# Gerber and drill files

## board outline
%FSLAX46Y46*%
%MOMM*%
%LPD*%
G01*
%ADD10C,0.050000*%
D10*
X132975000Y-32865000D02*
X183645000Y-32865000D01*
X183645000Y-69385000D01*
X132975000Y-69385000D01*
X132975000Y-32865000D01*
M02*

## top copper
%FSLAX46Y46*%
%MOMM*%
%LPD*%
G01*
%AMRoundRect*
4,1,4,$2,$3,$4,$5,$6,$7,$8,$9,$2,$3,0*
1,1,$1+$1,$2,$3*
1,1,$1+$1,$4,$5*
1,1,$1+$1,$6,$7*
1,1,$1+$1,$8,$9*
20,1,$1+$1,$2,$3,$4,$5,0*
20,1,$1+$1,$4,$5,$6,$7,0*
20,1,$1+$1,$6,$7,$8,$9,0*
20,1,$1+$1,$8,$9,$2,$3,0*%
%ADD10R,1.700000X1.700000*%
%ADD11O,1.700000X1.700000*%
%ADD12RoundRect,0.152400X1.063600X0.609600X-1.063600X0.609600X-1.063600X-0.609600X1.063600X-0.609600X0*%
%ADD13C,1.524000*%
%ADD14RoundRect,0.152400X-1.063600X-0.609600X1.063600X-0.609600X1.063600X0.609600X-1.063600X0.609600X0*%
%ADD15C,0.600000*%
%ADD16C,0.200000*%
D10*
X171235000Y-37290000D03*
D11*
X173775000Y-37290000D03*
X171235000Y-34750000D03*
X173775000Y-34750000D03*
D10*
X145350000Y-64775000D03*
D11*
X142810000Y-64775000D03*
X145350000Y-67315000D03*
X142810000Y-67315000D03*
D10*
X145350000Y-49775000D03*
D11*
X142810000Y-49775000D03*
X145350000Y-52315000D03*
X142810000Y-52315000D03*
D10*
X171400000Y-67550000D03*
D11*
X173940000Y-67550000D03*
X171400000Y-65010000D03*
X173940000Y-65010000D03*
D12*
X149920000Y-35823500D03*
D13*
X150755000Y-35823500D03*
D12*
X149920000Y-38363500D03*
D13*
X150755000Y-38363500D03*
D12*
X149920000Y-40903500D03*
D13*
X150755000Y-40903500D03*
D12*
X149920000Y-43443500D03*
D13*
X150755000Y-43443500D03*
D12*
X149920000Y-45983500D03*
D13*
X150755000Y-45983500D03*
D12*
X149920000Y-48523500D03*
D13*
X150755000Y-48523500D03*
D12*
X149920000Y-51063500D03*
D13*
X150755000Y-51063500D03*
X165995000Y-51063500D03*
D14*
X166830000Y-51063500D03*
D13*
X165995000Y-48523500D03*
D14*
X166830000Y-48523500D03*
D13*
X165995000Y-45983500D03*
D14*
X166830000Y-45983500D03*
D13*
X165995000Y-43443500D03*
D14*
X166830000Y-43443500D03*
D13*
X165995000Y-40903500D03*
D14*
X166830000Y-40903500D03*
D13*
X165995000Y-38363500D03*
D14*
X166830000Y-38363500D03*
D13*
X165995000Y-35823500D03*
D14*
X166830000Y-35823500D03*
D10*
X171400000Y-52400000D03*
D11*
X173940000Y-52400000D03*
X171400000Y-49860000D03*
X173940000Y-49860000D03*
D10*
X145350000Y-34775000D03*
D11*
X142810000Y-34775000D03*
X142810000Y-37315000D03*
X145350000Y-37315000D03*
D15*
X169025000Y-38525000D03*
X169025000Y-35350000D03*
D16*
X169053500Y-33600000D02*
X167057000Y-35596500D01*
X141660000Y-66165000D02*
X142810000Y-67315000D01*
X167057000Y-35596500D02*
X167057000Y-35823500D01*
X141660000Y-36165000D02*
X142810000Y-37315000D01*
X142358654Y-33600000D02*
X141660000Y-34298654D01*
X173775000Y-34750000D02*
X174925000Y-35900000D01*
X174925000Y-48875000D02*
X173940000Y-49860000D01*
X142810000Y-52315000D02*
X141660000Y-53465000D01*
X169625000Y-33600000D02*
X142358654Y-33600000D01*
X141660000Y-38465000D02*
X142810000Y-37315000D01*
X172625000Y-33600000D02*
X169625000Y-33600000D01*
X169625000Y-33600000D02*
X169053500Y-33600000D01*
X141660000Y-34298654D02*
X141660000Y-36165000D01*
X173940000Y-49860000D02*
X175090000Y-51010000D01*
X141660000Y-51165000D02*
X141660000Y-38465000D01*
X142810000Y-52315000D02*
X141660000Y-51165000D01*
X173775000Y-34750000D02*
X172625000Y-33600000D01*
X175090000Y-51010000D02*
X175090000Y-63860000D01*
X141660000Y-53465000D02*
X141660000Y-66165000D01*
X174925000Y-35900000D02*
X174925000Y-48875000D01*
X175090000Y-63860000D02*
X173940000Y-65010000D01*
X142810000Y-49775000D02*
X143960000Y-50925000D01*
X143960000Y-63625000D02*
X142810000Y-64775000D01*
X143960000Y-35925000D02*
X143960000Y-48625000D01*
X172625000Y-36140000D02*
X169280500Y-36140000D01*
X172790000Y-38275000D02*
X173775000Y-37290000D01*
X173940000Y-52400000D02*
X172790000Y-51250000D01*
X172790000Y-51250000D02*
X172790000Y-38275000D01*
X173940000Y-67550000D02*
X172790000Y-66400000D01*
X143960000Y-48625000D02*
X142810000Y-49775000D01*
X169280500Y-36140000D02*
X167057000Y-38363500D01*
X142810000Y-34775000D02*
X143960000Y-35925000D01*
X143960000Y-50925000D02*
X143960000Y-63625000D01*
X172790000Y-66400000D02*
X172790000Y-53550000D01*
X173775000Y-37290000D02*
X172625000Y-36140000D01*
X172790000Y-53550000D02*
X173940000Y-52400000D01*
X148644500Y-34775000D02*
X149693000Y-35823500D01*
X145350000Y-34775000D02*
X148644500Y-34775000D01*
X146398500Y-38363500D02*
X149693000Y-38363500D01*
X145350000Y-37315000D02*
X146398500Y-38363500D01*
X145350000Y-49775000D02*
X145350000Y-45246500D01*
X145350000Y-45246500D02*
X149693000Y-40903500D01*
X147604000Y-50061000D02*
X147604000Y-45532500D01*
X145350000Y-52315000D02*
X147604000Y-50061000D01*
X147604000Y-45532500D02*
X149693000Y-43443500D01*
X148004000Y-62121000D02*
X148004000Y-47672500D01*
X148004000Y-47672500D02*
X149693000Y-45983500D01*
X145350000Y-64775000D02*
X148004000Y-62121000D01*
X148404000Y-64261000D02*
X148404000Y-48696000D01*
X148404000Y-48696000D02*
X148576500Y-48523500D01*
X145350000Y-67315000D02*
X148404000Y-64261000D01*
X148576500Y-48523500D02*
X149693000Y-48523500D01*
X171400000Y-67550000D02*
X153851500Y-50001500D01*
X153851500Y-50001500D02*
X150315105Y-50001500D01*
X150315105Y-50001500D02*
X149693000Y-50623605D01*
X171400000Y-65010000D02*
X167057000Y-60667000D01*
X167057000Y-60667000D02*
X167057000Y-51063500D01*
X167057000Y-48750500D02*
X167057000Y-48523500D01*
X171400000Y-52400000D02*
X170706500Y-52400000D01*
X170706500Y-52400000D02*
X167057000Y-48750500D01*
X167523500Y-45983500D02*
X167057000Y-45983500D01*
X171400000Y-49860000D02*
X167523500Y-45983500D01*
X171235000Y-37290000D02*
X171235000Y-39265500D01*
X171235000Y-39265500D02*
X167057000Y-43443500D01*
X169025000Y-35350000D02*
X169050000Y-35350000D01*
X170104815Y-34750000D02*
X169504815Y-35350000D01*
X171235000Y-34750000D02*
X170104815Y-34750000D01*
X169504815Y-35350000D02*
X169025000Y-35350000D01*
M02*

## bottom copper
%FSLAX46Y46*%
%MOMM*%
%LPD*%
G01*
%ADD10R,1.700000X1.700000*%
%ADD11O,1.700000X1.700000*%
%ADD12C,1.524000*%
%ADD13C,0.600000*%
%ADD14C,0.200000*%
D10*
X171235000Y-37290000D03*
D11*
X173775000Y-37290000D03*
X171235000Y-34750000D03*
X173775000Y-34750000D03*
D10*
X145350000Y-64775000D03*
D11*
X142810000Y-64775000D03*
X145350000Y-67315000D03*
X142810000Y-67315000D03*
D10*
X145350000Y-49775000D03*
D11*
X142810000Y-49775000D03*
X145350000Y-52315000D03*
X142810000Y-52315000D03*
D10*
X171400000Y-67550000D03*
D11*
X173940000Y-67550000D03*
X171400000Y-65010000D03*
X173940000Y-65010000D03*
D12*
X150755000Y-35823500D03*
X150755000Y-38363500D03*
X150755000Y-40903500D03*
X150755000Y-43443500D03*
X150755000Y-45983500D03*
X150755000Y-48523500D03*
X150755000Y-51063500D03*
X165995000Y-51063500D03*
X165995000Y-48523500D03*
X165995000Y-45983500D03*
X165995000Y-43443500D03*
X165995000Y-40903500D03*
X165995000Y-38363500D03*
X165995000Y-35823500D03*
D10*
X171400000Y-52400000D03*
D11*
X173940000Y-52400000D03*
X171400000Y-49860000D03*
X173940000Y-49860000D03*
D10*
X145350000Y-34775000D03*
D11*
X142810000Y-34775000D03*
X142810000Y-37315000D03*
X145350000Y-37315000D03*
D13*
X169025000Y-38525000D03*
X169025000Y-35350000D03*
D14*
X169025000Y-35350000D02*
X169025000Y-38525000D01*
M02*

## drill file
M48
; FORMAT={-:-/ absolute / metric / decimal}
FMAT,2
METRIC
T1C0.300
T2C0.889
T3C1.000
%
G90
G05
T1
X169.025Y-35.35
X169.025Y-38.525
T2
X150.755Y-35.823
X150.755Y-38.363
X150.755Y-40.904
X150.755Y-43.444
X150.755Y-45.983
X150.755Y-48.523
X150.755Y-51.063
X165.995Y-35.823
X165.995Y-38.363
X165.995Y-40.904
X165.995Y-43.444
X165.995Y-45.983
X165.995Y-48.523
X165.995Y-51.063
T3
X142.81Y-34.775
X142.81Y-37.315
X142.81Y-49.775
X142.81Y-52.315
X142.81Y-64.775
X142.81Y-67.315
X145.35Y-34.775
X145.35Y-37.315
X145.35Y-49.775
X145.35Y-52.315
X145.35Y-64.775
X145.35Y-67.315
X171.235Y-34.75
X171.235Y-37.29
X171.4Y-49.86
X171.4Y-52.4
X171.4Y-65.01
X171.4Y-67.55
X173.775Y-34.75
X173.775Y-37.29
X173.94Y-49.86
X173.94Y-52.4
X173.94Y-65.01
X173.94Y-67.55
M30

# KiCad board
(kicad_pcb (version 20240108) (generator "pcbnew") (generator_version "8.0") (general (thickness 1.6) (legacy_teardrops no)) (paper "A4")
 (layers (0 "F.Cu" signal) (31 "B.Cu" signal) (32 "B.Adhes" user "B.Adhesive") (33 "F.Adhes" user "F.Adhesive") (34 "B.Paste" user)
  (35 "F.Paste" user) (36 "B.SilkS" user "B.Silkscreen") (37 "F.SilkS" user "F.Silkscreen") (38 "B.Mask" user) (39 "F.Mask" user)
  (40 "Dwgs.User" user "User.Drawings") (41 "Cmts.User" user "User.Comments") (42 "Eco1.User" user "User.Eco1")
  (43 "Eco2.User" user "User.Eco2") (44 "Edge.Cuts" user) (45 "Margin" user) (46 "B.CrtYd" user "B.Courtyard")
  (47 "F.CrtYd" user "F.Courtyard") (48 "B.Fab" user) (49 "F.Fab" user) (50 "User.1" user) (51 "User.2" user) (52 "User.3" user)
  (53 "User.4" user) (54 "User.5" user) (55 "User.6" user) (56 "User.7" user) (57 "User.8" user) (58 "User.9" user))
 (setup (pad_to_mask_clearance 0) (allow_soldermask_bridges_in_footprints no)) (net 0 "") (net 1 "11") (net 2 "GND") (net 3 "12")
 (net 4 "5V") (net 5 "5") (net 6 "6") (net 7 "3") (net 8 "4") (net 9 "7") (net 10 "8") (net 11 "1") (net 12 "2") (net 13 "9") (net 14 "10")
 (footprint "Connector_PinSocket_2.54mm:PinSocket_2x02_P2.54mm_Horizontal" (layer "F.Cu") (at 171.235 37.29 180)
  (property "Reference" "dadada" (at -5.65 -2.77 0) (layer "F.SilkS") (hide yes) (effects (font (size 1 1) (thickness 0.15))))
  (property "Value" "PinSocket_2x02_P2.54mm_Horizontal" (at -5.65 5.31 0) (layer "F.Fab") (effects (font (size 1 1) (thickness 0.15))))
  (pad "1" thru_hole rect (at 0 0 180) (size 1.7 1.7) (drill 1) (layers "*.Cu" "*.Mask") (remove_unused_layers no) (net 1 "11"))
  (pad "2" thru_hole oval (at -2.54 0 180) (size 1.7 1.7) (drill 1) (layers "*.Cu" "*.Mask") (remove_unused_layers no) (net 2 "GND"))
  (pad "3" thru_hole oval (at 0 2.54 180) (size 1.7 1.7) (drill 1) (layers "*.Cu" "*.Mask") (remove_unused_layers no) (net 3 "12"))
  (pad "4" thru_hole oval (at -2.54 2.54 180) (size 1.7 1.7) (drill 1) (layers "*.Cu" "*.Mask") (remove_unused_layers no) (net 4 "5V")))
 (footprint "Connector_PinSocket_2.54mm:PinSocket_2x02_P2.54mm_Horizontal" (layer "F.Cu") (at 145.35 64.775)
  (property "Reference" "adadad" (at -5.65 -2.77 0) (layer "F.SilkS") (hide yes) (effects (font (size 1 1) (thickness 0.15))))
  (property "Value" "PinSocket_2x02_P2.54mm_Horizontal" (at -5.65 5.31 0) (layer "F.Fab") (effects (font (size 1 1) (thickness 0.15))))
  (pad "1" thru_hole rect (at 0 0) (size 1.7 1.7) (drill 1) (layers "*.Cu" "*.Mask") (remove_unused_layers no) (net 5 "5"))
  (pad "2" thru_hole oval (at -2.54 0) (size 1.7 1.7) (drill 1) (layers "*.Cu" "*.Mask") (remove_unused_layers no) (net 2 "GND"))
  (pad "3" thru_hole oval (at 0 2.54) (size 1.7 1.7) (drill 1) (layers "*.Cu" "*.Mask") (remove_unused_layers no) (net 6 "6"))
  (pad "4" thru_hole oval (at -2.54 2.54) (size 1.7 1.7) (drill 1) (layers "*.Cu" "*.Mask") (remove_unused_layers no) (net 4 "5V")))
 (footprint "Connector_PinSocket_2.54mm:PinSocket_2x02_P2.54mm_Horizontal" (layer "F.Cu") (at 145.35 49.775)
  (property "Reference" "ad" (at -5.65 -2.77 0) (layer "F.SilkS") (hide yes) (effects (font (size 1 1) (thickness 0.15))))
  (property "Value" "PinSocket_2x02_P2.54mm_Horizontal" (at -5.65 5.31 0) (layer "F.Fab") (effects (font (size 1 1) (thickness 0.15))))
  (pad "1" thru_hole rect (at 0 0) (size 1.7 1.7) (drill 1) (layers "*.Cu" "*.Mask") (remove_unused_layers no) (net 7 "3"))
  (pad "2" thru_hole oval (at -2.54 0) (size 1.7 1.7) (drill 1) (layers "*.Cu" "*.Mask") (remove_unused_layers no) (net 2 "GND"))
  (pad "3" thru_hole oval (at 0 2.54) (size 1.7 1.7) (drill 1) (layers "*.Cu" "*.Mask") (remove_unused_layers no) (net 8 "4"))
  (pad "4" thru_hole oval (at -2.54 2.54) (size 1.7 1.7) (drill 1) (layers "*.Cu" "*.Mask") (remove_unused_layers no) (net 4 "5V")))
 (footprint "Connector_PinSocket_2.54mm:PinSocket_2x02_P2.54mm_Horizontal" (layer "F.Cu") (at 171.4 67.55 180)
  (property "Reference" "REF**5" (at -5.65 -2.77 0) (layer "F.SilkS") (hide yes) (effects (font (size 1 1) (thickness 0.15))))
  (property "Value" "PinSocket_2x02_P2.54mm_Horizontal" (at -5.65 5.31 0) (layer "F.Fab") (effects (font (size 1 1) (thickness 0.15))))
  (pad "1" thru_hole rect (at 0 0 180) (size 1.7 1.7) (drill 1) (layers "*.Cu" "*.Mask") (remove_unused_layers no) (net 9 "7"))
  (pad "2" thru_hole oval (at -2.54 0 180) (size 1.7 1.7) (drill 1) (layers "*.Cu" "*.Mask") (remove_unused_layers no) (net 2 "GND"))
  (pad "3" thru_hole oval (at 0 2.54 180) (size 1.7 1.7) (drill 1) (layers "*.Cu" "*.Mask") (remove_unused_layers no) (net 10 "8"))
  (pad "4" thru_hole oval (at -2.54 2.54 180) (size 1.7 1.7) (drill 1) (layers "*.Cu" "*.Mask" "B.Paste") (remove_unused_layers no)
   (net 4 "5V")))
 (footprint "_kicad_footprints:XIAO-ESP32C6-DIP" (layer "F.Cu") (at 158.42 43.4435)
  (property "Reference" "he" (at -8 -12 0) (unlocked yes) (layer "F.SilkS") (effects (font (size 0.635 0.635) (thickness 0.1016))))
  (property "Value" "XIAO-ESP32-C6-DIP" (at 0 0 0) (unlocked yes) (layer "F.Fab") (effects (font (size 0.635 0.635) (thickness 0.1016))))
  (pad "1" smd roundrect (at -8.5 -7.62 180) (size 2.432 1.524) (layers "F.Cu" "F.Mask") (roundrect_rratio 0.1) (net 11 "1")
   (thermal_bridge_angle 45))
  (pad "1" thru_hole circle (at -7.665 -7.62 180) (size 1.524 1.524) (drill 0.889) (layers "*.Cu" "*.Mask") (remove_unused_layers no))
  (pad "2" smd roundrect (at -8.5 -5.08 180) (size 2.432 1.524) (layers "F.Cu" "F.Mask") (roundrect_rratio 0.1) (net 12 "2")
   (thermal_bridge_angle 45))
  (pad "2" thru_hole circle (at -7.665 -5.08 180) (size 1.524 1.524) (drill 0.889) (layers "*.Cu" "*.Mask") (remove_unused_layers no))
  (pad "3" smd roundrect (at -8.5 -2.54 180) (size 2.432 1.524) (layers "F.Cu" "F.Mask") (roundrect_rratio 0.1) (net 7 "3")
   (thermal_bridge_angle 45))
  (pad "3" thru_hole circle (at -7.665 -2.54 180) (size 1.524 1.524) (drill 0.889) (layers "*.Cu" "*.Mask") (remove_unused_layers no))
  (pad "4" smd roundrect (at -8.5 0 180) (size 2.432 1.524) (layers "F.Cu" "F.Mask") (roundrect_rratio 0.1) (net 8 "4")
   (thermal_bridge_angle 45))
  (pad "4" thru_hole circle (at -7.665 0 180) (size 1.524 1.524) (drill 0.889) (layers "*.Cu" "*.Mask") (remove_unused_layers no))
  (pad "5" smd roundrect (at -8.5 2.54 180) (size 2.432 1.524) (layers "F.Cu" "F.Mask") (roundrect_rratio 0.1) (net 5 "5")
   (thermal_bridge_angle 45))
  (pad "5" thru_hole circle (at -7.665 2.54 180) (size 1.524 1.524) (drill 0.889) (layers "*.Cu" "*.Mask") (remove_unused_layers no))
  (pad "6" smd roundrect (at -8.5 5.08 180) (size 2.432 1.524) (layers "F.Cu" "F.Mask") (roundrect_rratio 0.1) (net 6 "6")
   (thermal_bridge_angle 45))
  (pad "6" thru_hole circle (at -7.665 5.08 180) (size 1.524 1.524) (drill 0.889) (layers "*.Cu" "*.Mask") (remove_unused_layers no))
  (pad "7" smd roundrect (at -8.5 7.62 180) (size 2.432 1.524) (layers "F.Cu" "F.Mask") (roundrect_rratio 0.1) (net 9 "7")
   (thermal_bridge_angle 45))
  (pad "7" thru_hole circle (at -7.665 7.62 180) (size 1.524 1.524) (drill 0.889) (layers "*.Cu" "*.Mask") (remove_unused_layers no))
  (pad "8" thru_hole circle (at 7.575 7.62) (size 1.524 1.524) (drill 0.889) (layers "*.Cu" "*.Mask") (remove_unused_layers no))
  (pad "8" smd roundrect (at 8.41 7.62) (size 2.432 1.524) (layers "F.Cu" "F.Mask") (roundrect_rratio 0.1) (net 10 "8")
   (thermal_bridge_angle 45))
  (pad "9" thru_hole circle (at 7.575 5.08) (size 1.524 1.524) (drill 0.889) (layers "*.Cu" "*.Mask") (remove_unused_layers no))
  (pad "9" smd roundrect (at 8.41 5.08) (size 2.432 1.524) (layers "F.Cu" "F.Mask") (roundrect_rratio 0.1) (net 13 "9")
   (thermal_bridge_angle 45))
  (pad "10" thru_hole circle (at 7.575 2.54) (size 1.524 1.524) (drill 0.889) (layers "*.Cu" "*.Mask") (remove_unused_layers no))
  (pad "10" smd roundrect (at 8.41 2.54) (size 2.432 1.524) (layers "F.Cu" "F.Mask") (roundrect_rratio 0.1) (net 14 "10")
   (thermal_bridge_angle 45))
  (pad "11" thru_hole circle (at 7.575 0) (size 1.524 1.524) (drill 0.889) (layers "*.Cu" "*.Mask") (remove_unused_layers no))
  (pad "11" smd roundrect (at 8.41 0) (size 2.432 1.524) (layers "F.Cu" "F.Mask") (roundrect_rratio 0.1) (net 1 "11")
   (thermal_bridge_angle 45))
  (pad "12" thru_hole circle (at 7.575 -2.54) (size 1.524 1.524) (drill 0.889) (layers "*.Cu" "*.Mask") (remove_unused_layers no))
  (pad "12" smd roundrect (at 8.41 -2.54) (size 2.432 1.524) (layers "F.Cu" "F.Mask") (roundrect_rratio 0.1) (thermal_bridge_angle 45))
  (pad "13" thru_hole circle (at 7.575 -5.08) (size 1.524 1.524) (drill 0.889) (layers "*.Cu" "*.Mask") (remove_unused_layers no))
  (pad "13" smd roundrect (at 8.41 -5.08) (size 2.432 1.524) (layers "F.Cu" "F.Mask") (roundrect_rratio 0.1) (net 2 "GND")
   (thermal_bridge_angle 45))
  (pad "14" thru_hole circle (at 7.575 -7.62) (size 1.524 1.524) (drill 0.889) (layers "*.Cu" "*.Mask") (remove_unused_layers no))
  (pad "14" smd roundrect (at 8.41 -7.62) (size 2.432 1.524) (layers "F.Cu" "F.Mask") (roundrect_rratio 0.1) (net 4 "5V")
   (thermal_bridge_angle 45)))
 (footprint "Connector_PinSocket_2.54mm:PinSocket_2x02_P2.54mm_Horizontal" (layer "F.Cu") (at 171.4 52.4 180)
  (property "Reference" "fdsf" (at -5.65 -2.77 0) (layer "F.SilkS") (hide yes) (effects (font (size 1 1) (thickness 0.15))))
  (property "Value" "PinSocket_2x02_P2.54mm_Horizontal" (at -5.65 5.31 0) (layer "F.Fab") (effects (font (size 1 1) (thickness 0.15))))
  (pad "1" thru_hole rect (at 0 0 180) (size 1.7 1.7) (drill 1) (layers "*.Cu" "*.Mask") (remove_unused_layers no) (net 13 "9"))
  (pad "2" thru_hole oval (at -2.54 0 180) (size 1.7 1.7) (drill 1) (layers "*.Cu" "*.Mask") (remove_unused_layers no) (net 2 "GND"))
  (pad "3" thru_hole oval (at 0 2.54 180) (size 1.7 1.7) (drill 1) (layers "*.Cu" "*.Mask") (remove_unused_layers no) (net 14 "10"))
  (pad "4" thru_hole oval (at -2.54 2.54 180) (size 1.7 1.7) (drill 1) (layers "*.Cu" "*.Mask") (remove_unused_layers no) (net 4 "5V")))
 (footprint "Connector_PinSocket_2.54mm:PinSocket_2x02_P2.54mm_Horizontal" (layer "F.Cu") (at 145.35 34.775)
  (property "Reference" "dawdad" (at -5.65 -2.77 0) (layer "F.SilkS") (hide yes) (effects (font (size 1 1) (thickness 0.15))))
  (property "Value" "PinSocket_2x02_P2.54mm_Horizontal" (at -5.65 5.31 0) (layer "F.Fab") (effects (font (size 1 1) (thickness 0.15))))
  (pad "1" thru_hole rect (at 0 0) (size 1.7 1.7) (drill 1) (layers "*.Cu" "*.Mask") (remove_unused_layers no) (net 11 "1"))
  (pad "2" thru_hole oval (at -2.54 0) (size 1.7 1.7) (drill 1) (layers "*.Cu" "*.Mask") (remove_unused_layers no) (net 2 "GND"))
  (pad "2" thru_hole oval (at -2.54 2.54) (size 1.7 1.7) (drill 1) (layers "*.Cu" "*.Mask") (remove_unused_layers no) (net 4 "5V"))
  (pad "eeeeee" thru_hole oval (at 0 2.54) (size 1.7 1.7) (drill 1) (layers "*.Cu" "*.Mask") (remove_unused_layers no) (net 12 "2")))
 (gr_rect (start 132.975 32.865) (end 183.645 69.385) (stroke (width 0.05) (type default)) (fill none) (layer "Edge.Cuts"))
 (segment (start 169.0535 33.6) (end 167.057 35.5965) (width 0.2) (layer "F.Cu") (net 4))
 (segment (start 141.66 66.165) (end 142.81 67.315) (width 0.2) (layer "F.Cu") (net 4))
 (segment (start 167.057 35.5965) (end 167.057 35.8235) (width 0.2) (layer "F.Cu") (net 4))
 (segment (start 141.66 36.165) (end 142.81 37.315) (width 0.2) (layer "F.Cu") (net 4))
 (segment (start 142.358654 33.6) (end 141.66 34.298654) (width 0.2) (layer "F.Cu") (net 4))
 (segment (start 173.775 34.75) (end 174.925 35.9) (width 0.2) (layer "F.Cu") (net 4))
 (segment (start 174.925 48.875) (end 173.94 49.86) (width 0.2) (layer "F.Cu") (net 4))
 (segment (start 142.81 52.315) (end 141.66 53.465) (width 0.2) (layer "F.Cu") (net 4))
 (segment (start 169.625 33.6) (end 142.358654 33.6) (width 0.2) (layer "F.Cu") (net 4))
 (segment (start 141.66 38.465) (end 142.81 37.315) (width 0.2) (layer "F.Cu") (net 4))
 (segment (start 172.625 33.6) (end 169.625 33.6) (width 0.2) (layer "F.Cu") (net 4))
 (segment (start 169.625 33.6) (end 169.0535 33.6) (width 0.2) (layer "F.Cu") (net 4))
 (segment (start 141.66 34.298654) (end 141.66 36.165) (width 0.2) (layer "F.Cu") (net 4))
 (segment (start 173.94 49.86) (end 175.09 51.01) (width 0.2) (layer "F.Cu") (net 4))
 (segment (start 141.66 51.165) (end 141.66 38.465) (width 0.2) (layer "F.Cu") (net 4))
 (segment (start 142.81 52.315) (end 141.66 51.165) (width 0.2) (layer "F.Cu") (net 4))
 (segment (start 173.775 34.75) (end 172.625 33.6) (width 0.2) (layer "F.Cu") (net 4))
 (segment (start 175.09 51.01) (end 175.09 63.86) (width 0.2) (layer "F.Cu") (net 4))
 (segment (start 141.66 53.465) (end 141.66 66.165) (width 0.2) (layer "F.Cu") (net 4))
 (segment (start 174.925 35.9) (end 174.925 48.875) (width 0.2) (layer "F.Cu") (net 4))
 (segment (start 175.09 63.86) (end 173.94 65.01) (width 0.2) (layer "F.Cu") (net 4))
 (segment (start 142.81 49.775) (end 143.96 50.925) (width 0.2) (layer "F.Cu") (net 2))
 (segment (start 143.96 63.625) (end 142.81 64.775) (width 0.2) (layer "F.Cu") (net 2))
 (segment (start 143.96 35.925) (end 143.96 48.625) (width 0.2) (layer "F.Cu") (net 2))
 (segment (start 172.625 36.14) (end 169.2805 36.14) (width 0.2) (layer "F.Cu") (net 2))
 (segment (start 172.79 38.275) (end 173.775 37.29) (width 0.2) (layer "F.Cu") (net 2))
 (segment (start 173.94 52.4) (end 172.79 51.25) (width 0.2) (layer "F.Cu") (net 2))
 (segment (start 172.79 51.25) (end 172.79 38.275) (width 0.2) (layer "F.Cu") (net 2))
 (segment (start 173.94 67.55) (end 172.79 66.4) (width 0.2) (layer "F.Cu") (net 2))
 (segment (start 143.96 48.625) (end 142.81 49.775) (width 0.2) (layer "F.Cu") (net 2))
 (segment (start 169.2805 36.14) (end 167.057 38.3635) (width 0.2) (layer "F.Cu") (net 2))
 (segment (start 142.81 34.775) (end 143.96 35.925) (width 0.2) (layer "F.Cu") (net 2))
 (segment (start 143.96 50.925) (end 143.96 63.625) (width 0.2) (layer "F.Cu") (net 2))
 (segment (start 172.79 66.4) (end 172.79 53.55) (width 0.2) (layer "F.Cu") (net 2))
 (segment (start 173.775 37.29) (end 172.625 36.14) (width 0.2) (layer "F.Cu") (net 2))
 (segment (start 172.79 53.55) (end 173.94 52.4) (width 0.2) (layer "F.Cu") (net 2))
 (segment (start 148.6445 34.775) (end 149.693 35.8235) (width 0.2) (layer "F.Cu") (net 11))
 (segment (start 145.35 34.775) (end 148.6445 34.775) (width 0.2) (layer "F.Cu") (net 11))
 (segment (start 146.3985 38.3635) (end 149.693 38.3635) (width 0.2) (layer "F.Cu") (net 12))
 (segment (start 145.35 37.315) (end 146.3985 38.3635) (width 0.2) (layer "F.Cu") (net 12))
 (segment (start 145.35 49.775) (end 145.35 45.2465) (width 0.2) (layer "F.Cu") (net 7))
 (segment (start 145.35 45.2465) (end 149.693 40.9035) (width 0.2) (layer "F.Cu") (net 7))
 (segment (start 147.604 50.061) (end 147.604 45.5325) (width 0.2) (layer "F.Cu") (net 8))
 (segment (start 145.35 52.315) (end 147.604 50.061) (width 0.2) (layer "F.Cu") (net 8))
 (segment (start 147.604 45.5325) (end 149.693 43.4435) (width 0.2) (layer "F.Cu") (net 8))
 (segment (start 148.004 62.121) (end 148.004 47.6725) (width 0.2) (layer "F.Cu") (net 5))
 (segment (start 148.004 47.6725) (end 149.693 45.9835) (width 0.2) (layer "F.Cu") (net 5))
 (segment (start 145.35 64.775) (end 148.004 62.121) (width 0.2) (layer "F.Cu") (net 5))
 (segment (start 148.404 64.261) (end 148.404 48.696) (width 0.2) (layer "F.Cu") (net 6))
 (segment (start 148.404 48.696) (end 148.5765 48.5235) (width 0.2) (layer "F.Cu") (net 6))
 (segment (start 145.35 67.315) (end 148.404 64.261) (width 0.2) (layer "F.Cu") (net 6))
 (segment (start 148.5765 48.5235) (end 149.693 48.5235) (width 0.2) (layer "F.Cu") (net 6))
 (segment (start 171.4 67.55) (end 153.8515 50.0015) (width 0.2) (layer "F.Cu") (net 9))
 (segment (start 153.8515 50.0015) (end 150.315105 50.0015) (width 0.2) (layer "F.Cu") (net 9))
 (segment (start 150.315105 50.0015) (end 149.693 50.623605) (width 0.2) (layer "F.Cu") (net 9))
 (segment (start 171.4 65.01) (end 167.057 60.667) (width 0.2) (layer "F.Cu") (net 10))
 (segment (start 167.057 60.667) (end 167.057 51.0635) (width 0.2) (layer "F.Cu") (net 10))
 (segment (start 167.057 48.7505) (end 167.057 48.5235) (width 0.2) (layer "F.Cu") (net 13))
 (segment (start 171.4 52.4) (end 170.7065 52.4) (width 0.2) (layer "F.Cu") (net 13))
 (segment (start 170.7065 52.4) (end 167.057 48.7505) (width 0.2) (layer "F.Cu") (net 13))
 (segment (start 167.5235 45.9835) (end 167.057 45.9835) (width 0.2) (layer "F.Cu") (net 14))
 (segment (start 171.4 49.86) (end 167.5235 45.9835) (width 0.2) (layer "F.Cu") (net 14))
 (segment (start 171.235 37.29) (end 171.235 39.2655) (width 0.2) (layer "F.Cu") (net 1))
 (segment (start 171.235 39.2655) (end 167.057 43.4435) (width 0.2) (layer "F.Cu") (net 1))
 (segment (start 169.025 35.35) (end 169.05 35.35) (width 0.2) (layer "F.Cu") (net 3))
 (segment (start 170.104815 34.75) (end 169.504815 35.35) (width 0.2) (layer "F.Cu") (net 3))
 (segment (start 171.235 34.75) (end 170.104815 34.75) (width 0.2) (layer "F.Cu") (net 3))
 (segment (start 169.504815 35.35) (end 169.025 35.35) (width 0.2) (layer "F.Cu") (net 3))
 (via (at 169.025 38.525) (size 0.6) (drill 0.3) (layers "F.Cu" "B.Cu") (free yes) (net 3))
 (via (at 169.025 35.35) (size 0.6) (drill 0.3) (layers "F.Cu" "B.Cu") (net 3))
 (segment (start 169.025 35.35) (end 169.025 38.525) (width 0.2) (layer "B.Cu") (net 3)))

